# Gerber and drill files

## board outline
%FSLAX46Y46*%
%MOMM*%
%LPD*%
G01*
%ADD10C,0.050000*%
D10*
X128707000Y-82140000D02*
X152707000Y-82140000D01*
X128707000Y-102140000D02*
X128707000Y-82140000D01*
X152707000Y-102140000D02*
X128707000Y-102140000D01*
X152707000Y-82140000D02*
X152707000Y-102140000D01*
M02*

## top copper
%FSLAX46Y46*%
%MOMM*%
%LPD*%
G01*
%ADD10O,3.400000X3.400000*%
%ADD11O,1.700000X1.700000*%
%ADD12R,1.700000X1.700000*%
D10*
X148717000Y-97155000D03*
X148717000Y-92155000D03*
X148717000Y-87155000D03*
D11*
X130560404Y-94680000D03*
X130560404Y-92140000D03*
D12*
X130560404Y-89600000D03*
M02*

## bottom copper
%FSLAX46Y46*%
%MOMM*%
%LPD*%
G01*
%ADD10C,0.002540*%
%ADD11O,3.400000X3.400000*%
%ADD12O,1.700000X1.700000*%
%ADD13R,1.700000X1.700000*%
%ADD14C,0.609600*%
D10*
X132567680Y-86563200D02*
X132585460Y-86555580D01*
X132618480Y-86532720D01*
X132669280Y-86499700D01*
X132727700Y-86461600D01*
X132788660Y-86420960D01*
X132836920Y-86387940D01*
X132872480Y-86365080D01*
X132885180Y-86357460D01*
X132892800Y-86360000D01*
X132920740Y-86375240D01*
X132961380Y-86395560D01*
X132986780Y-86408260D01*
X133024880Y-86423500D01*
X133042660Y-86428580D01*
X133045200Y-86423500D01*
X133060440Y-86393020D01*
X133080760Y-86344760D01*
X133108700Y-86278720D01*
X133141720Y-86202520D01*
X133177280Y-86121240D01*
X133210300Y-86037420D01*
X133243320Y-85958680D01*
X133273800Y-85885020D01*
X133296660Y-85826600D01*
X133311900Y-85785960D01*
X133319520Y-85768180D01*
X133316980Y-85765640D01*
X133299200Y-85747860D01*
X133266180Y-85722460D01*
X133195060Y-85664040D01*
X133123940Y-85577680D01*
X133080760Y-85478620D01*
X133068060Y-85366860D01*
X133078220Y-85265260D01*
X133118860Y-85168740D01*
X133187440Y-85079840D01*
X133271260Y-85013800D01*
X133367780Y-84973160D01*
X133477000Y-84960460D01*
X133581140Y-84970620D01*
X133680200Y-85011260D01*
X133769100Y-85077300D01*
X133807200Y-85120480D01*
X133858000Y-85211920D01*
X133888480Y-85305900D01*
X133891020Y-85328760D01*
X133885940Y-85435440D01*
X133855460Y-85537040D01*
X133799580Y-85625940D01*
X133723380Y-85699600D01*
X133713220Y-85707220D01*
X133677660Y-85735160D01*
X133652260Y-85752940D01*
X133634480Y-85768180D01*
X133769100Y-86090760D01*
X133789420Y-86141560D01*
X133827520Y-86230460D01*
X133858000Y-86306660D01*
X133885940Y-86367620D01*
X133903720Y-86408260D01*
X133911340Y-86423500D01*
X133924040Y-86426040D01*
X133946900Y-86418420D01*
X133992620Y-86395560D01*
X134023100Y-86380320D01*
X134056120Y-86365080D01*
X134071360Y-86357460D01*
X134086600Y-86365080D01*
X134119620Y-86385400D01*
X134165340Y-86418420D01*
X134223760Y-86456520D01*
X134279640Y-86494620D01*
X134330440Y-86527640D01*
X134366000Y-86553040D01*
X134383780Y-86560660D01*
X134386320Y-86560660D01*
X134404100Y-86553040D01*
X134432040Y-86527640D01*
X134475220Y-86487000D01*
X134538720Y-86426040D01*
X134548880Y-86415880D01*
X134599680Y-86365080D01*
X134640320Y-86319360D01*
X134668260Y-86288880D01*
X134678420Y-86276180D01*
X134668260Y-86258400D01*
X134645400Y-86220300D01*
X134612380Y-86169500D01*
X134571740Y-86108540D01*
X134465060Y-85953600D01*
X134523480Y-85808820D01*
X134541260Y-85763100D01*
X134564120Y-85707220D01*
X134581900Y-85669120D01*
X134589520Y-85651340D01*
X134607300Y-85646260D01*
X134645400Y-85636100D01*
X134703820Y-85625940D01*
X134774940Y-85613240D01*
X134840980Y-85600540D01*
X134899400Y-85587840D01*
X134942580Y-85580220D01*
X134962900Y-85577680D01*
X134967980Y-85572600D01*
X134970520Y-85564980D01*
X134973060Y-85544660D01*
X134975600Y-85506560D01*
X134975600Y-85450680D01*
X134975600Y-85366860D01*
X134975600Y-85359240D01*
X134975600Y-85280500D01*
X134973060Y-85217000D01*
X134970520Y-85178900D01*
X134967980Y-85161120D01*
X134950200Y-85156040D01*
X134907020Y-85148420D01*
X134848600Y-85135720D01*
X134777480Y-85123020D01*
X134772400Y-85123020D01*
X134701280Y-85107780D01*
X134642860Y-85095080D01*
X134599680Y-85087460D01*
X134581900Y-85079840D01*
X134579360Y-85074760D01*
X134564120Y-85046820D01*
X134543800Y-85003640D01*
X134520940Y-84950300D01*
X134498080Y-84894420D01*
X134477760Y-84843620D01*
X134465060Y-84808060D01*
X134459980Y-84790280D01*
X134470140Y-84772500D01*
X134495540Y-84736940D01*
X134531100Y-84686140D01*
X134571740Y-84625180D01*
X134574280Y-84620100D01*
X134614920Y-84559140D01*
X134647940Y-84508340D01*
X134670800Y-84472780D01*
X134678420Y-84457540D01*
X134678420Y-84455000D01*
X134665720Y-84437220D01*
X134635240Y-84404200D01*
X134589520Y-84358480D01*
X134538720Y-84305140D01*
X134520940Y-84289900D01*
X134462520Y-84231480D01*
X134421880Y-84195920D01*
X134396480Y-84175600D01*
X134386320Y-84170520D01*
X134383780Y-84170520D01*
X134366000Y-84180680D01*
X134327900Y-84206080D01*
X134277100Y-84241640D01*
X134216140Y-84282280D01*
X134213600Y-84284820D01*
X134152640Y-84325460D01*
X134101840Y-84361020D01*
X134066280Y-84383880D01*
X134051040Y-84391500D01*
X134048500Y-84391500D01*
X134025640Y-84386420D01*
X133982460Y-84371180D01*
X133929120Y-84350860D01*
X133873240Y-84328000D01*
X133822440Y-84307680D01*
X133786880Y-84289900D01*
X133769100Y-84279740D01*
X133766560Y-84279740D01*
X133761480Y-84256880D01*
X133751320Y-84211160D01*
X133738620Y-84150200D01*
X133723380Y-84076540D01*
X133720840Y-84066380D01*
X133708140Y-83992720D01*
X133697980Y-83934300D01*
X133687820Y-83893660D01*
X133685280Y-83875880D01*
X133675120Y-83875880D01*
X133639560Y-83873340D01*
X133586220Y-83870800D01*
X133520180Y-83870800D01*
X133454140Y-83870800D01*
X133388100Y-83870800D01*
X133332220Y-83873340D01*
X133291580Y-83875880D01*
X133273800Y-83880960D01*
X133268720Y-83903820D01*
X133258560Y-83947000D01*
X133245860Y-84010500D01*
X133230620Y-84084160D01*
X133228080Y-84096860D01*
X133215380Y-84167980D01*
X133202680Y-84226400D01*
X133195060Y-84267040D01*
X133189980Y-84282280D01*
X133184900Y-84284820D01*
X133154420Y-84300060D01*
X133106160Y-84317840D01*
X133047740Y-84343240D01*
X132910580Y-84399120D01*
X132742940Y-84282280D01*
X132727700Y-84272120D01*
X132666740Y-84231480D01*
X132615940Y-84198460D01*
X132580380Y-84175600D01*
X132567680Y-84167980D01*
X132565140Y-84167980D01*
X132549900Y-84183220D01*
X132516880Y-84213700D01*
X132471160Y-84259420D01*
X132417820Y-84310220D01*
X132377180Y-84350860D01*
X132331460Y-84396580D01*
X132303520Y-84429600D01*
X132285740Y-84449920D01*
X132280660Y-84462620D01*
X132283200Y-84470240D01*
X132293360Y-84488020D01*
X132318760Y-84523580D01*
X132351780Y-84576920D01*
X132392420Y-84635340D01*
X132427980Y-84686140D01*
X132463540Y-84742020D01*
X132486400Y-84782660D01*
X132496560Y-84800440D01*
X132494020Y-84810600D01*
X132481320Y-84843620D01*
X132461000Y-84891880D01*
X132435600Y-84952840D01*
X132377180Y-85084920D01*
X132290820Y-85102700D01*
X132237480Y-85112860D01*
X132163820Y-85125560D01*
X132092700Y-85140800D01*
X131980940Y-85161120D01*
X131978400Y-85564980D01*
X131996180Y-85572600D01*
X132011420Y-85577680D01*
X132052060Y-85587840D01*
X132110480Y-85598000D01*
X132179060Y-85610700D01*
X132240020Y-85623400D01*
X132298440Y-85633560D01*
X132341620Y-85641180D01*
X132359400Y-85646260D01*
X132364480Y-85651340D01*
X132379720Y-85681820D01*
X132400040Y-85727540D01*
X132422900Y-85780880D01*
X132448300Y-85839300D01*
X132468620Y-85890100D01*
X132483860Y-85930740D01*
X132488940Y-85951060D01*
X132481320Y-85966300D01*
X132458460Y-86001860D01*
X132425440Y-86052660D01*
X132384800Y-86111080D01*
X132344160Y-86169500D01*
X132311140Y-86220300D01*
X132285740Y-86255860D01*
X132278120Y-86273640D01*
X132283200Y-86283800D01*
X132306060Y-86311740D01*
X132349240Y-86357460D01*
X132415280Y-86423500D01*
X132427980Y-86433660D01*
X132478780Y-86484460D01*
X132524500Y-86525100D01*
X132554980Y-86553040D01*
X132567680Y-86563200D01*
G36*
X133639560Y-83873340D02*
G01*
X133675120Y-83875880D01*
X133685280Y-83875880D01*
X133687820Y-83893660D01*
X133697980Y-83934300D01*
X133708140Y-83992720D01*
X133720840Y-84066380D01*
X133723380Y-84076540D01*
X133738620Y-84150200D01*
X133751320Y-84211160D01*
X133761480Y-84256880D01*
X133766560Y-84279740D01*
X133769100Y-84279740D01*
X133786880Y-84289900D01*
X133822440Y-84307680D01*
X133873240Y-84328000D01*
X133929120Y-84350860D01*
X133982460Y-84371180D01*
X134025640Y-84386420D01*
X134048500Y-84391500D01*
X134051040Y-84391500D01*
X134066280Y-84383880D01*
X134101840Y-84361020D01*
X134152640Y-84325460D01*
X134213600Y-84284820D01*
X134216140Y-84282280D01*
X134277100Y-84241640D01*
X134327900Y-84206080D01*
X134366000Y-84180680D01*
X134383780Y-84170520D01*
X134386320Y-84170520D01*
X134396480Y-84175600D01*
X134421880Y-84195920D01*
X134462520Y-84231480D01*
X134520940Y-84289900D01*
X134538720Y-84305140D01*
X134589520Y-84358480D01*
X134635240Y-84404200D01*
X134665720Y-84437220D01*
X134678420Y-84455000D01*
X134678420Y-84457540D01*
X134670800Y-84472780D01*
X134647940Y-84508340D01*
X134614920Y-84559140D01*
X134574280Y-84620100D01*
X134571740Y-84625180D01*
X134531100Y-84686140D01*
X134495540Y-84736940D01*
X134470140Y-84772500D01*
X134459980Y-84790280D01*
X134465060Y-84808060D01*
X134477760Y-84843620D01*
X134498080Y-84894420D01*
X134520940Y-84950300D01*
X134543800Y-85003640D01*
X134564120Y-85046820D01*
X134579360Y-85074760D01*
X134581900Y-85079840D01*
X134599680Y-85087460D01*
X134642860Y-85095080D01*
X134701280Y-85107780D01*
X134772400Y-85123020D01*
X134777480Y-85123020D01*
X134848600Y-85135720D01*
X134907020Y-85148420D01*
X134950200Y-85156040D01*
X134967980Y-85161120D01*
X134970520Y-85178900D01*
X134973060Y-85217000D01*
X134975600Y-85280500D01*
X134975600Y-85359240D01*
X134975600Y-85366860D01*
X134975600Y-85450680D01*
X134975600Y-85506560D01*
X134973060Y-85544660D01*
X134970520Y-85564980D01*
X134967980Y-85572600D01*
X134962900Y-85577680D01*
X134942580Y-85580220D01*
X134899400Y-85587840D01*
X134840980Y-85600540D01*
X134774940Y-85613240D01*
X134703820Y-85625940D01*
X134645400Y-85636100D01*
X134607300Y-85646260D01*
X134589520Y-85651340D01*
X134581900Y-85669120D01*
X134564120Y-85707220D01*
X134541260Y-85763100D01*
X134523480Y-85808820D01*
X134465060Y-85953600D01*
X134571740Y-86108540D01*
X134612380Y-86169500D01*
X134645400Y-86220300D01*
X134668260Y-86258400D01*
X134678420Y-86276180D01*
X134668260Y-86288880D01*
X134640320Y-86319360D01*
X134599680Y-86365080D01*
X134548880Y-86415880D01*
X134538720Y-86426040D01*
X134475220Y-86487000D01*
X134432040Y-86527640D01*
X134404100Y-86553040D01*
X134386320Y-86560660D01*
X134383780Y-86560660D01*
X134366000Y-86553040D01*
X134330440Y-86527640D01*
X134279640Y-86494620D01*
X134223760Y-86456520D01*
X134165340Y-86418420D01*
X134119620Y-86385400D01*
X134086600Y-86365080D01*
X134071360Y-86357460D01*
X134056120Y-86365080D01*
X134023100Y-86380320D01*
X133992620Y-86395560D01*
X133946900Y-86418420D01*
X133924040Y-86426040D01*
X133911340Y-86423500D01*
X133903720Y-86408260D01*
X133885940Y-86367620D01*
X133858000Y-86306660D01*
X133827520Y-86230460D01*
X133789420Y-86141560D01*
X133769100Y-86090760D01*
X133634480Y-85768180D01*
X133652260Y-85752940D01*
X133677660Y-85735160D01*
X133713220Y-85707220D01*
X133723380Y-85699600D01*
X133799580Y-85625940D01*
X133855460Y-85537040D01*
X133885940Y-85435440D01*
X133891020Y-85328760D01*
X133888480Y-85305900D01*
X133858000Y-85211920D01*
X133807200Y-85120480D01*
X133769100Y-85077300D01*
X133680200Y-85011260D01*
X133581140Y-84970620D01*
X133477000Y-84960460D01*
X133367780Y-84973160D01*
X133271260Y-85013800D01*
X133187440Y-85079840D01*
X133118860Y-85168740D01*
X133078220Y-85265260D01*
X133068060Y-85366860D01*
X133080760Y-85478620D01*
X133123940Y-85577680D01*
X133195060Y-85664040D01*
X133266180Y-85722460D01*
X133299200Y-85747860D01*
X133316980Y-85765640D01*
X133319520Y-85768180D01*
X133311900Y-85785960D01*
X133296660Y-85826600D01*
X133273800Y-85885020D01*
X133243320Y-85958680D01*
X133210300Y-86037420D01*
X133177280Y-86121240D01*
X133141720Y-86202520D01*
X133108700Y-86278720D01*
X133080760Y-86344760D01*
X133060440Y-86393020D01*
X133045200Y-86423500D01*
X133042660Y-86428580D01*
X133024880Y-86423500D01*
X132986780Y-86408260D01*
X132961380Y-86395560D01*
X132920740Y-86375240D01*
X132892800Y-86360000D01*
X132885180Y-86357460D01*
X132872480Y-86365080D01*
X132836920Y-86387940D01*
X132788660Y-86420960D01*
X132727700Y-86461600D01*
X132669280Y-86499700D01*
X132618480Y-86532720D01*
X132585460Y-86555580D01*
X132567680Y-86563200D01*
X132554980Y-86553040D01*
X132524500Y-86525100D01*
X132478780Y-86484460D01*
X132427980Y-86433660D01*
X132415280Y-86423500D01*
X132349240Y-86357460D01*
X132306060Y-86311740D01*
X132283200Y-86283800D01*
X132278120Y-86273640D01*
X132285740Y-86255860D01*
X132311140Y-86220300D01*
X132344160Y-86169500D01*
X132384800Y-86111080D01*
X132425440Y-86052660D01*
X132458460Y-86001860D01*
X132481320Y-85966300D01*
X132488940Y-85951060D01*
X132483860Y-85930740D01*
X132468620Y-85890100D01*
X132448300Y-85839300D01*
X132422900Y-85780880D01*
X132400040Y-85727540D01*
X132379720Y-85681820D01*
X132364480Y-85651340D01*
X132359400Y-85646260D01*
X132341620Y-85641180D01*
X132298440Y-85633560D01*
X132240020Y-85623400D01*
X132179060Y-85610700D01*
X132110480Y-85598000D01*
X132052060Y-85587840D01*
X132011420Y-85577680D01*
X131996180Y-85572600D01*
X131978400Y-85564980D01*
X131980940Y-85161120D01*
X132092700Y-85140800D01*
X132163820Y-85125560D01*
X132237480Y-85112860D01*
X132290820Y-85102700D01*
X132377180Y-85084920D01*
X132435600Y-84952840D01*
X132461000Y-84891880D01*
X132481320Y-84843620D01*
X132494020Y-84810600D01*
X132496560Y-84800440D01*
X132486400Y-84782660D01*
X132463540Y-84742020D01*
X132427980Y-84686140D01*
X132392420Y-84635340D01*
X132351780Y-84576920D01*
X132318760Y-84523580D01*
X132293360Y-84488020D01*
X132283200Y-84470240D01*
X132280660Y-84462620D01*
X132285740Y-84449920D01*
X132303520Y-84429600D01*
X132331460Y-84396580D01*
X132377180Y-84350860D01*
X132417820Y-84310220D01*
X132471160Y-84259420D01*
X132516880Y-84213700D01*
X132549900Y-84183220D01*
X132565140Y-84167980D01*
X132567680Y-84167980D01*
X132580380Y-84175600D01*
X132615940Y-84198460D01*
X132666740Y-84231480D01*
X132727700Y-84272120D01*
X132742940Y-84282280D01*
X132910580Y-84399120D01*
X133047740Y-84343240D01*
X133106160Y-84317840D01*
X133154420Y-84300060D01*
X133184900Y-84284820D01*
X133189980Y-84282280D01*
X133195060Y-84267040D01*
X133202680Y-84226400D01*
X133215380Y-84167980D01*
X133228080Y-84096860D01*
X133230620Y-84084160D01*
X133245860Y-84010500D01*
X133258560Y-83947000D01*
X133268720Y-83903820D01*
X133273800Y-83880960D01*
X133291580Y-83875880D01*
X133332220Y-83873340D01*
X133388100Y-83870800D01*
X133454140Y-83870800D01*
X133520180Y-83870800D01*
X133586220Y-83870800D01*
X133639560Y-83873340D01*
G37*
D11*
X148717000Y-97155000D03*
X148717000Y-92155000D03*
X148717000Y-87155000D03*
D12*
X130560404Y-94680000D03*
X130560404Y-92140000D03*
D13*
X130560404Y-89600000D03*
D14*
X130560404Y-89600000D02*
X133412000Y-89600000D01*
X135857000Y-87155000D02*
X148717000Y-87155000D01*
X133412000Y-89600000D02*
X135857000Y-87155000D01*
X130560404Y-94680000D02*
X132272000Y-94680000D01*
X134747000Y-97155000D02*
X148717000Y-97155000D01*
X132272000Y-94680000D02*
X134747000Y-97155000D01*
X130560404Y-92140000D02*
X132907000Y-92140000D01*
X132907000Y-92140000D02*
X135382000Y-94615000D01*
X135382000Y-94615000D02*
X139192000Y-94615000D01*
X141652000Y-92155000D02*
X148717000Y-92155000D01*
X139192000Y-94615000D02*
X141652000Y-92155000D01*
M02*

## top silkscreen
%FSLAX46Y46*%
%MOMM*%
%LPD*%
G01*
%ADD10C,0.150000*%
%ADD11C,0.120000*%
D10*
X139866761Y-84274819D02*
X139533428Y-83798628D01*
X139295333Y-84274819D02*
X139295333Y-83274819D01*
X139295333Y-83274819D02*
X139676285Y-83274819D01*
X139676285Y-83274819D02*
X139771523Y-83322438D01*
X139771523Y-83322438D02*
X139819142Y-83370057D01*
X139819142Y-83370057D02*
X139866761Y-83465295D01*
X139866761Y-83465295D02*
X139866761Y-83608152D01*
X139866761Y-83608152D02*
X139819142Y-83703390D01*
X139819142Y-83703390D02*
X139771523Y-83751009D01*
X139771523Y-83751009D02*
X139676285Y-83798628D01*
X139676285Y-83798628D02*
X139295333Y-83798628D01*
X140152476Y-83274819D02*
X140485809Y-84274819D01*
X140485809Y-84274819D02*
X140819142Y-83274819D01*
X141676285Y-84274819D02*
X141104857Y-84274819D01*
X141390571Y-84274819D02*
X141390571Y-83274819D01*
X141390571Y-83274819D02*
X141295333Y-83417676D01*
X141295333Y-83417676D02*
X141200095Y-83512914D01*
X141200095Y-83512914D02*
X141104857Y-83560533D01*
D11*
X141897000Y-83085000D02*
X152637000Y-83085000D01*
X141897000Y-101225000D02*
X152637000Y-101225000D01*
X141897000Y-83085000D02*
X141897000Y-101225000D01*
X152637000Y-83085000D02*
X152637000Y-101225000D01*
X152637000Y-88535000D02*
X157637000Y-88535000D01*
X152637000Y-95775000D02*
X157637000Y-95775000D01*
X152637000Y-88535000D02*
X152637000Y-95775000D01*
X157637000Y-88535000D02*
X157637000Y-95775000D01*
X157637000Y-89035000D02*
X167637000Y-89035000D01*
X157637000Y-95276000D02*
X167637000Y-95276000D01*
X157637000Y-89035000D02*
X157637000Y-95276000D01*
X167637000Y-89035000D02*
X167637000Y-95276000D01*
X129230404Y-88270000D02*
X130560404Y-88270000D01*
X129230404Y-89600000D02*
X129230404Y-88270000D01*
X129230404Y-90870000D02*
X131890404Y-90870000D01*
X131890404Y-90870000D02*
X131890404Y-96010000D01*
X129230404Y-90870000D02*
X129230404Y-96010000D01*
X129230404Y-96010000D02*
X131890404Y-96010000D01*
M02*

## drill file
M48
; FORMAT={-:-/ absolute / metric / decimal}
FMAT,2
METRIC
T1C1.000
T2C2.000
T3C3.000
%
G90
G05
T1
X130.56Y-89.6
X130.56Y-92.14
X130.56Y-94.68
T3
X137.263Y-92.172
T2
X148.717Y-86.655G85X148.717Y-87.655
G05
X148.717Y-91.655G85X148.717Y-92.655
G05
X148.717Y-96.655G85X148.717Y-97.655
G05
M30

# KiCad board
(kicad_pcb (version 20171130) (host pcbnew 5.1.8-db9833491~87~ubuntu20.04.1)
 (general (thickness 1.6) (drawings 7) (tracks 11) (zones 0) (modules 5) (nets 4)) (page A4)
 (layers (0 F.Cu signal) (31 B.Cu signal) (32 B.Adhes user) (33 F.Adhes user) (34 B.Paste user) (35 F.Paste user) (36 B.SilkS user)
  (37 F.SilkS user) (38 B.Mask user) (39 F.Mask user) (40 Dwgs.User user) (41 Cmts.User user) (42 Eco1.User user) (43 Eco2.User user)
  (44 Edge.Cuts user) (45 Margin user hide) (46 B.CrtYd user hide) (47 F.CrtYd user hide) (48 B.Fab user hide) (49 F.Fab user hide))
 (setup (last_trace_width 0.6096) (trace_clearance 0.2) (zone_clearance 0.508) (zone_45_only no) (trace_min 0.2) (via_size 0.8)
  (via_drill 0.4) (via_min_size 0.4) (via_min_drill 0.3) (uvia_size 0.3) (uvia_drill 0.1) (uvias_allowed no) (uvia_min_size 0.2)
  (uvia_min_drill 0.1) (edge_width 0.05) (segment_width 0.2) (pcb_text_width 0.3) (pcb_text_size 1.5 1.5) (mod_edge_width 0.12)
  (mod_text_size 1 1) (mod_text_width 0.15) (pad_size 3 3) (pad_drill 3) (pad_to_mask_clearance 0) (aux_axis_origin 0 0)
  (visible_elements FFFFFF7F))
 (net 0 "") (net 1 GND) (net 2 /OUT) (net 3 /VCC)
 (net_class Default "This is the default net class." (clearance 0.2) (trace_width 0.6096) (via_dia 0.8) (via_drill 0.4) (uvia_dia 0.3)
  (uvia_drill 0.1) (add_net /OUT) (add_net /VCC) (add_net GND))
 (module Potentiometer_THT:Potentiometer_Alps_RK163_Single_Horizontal (layer F.Cu) (at 148.717 97.155)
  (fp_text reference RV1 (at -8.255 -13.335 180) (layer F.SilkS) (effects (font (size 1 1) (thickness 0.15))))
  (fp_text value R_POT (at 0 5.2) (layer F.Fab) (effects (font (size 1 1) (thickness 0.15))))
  (fp_line (start -6.82 -14.07) (end 3.92 -14.07) (layer F.SilkS) (width 0.12))
  (fp_line (start -6.82 4.07) (end 3.92 4.07) (layer F.SilkS) (width 0.12))
  (fp_line (start -6.82 -14.07) (end -6.82 4.07) (layer F.SilkS) (width 0.12))
  (fp_line (start 3.92 -14.07) (end 3.92 4.07) (layer F.SilkS) (width 0.12))
  (fp_line (start 3.92 -8.62) (end 8.92 -8.62) (layer F.SilkS) (width 0.12))
  (fp_line (start 3.92 -1.38) (end 8.92 -1.38) (layer F.SilkS) (width 0.12))
  (fp_line (start 3.92 -8.62) (end 3.92 -1.38) (layer F.SilkS) (width 0.12))
  (fp_line (start 8.92 -8.62) (end 8.92 -1.38) (layer F.SilkS) (width 0.12))
  (fp_line (start 8.92 -8.12) (end 18.92 -8.12) (layer F.SilkS) (width 0.12))
  (fp_line (start 8.92 -1.879) (end 18.92 -1.879) (layer F.SilkS) (width 0.12))
  (fp_line (start 8.92 -8.12) (end 8.92 -1.879) (layer F.SilkS) (width 0.12))
  (fp_line (start 18.92 -8.12) (end 18.92 -1.879) (layer F.SilkS) (width 0.12))
  (pad 1 thru_hole oval (at 0 0) (size 3.4 3.4) (drill oval 2 3) (layers *.Cu *.Mask) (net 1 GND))
  (pad 2 thru_hole oval (at 0 -5) (size 3.4 3.4) (drill oval 2 3) (layers *.Cu *.Mask) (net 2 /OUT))
  (pad 3 thru_hole oval (at 0 -10) (size 3.4 3.4) (drill oval 2 3) (layers *.Cu *.Mask) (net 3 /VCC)))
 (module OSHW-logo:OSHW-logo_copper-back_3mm (layer B.Cu) (at 133.477 85.217 180)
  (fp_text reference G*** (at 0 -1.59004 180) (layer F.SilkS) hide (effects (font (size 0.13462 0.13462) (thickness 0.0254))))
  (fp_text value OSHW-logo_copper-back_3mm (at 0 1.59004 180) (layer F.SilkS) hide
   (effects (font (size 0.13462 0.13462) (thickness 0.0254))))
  (fp_poly
   (pts (xy 0.90932 -1.3462) (xy 0.89154 -1.33858) (xy 0.85852 -1.31572) (xy 0.80772 -1.2827) (xy 0.7493 -1.2446) (xy 0.68834 -1.20396)
    (xy 0.64008 -1.17094) (xy 0.60452 -1.14808) (xy 0.59182 -1.14046) (xy 0.5842 -1.143) (xy 0.55626 -1.15824) (xy 0.51562 -1.17856)
    (xy 0.49022 -1.19126) (xy 0.45212 -1.2065) (xy 0.43434 -1.21158) (xy 0.4318 -1.2065) (xy 0.41656 -1.17602) (xy 0.39624 -1.12776)
    (xy 0.3683 -1.06172) (xy 0.33528 -0.98552) (xy 0.29972 -0.90424) (xy 0.2667 -0.82042) (xy 0.23368 -0.74168) (xy 0.2032 -0.66802)
    (xy 0.18034 -0.6096) (xy 0.1651 -0.56896) (xy 0.15748 -0.55118) (xy 0.16002 -0.54864) (xy 0.1778 -0.53086) (xy 0.21082 -0.50546)
    (xy 0.28194 -0.44704) (xy 0.35306 -0.36068) (xy 0.39624 -0.26162) (xy 0.40894 -0.14986) (xy 0.39878 -0.04826) (xy 0.35814 0.04826)
    (xy 0.28956 0.13716) (xy 0.20574 0.2032) (xy 0.10922 0.24384) (xy 0 0.25654) (xy -0.10414 0.24638) (xy -0.2032 0.20574)
    (xy -0.2921 0.1397) (xy -0.3302 0.09652) (xy -0.381 0.00508) (xy -0.41148 -0.0889) (xy -0.41402 -0.11176) (xy -0.40894 -0.21844)
    (xy -0.37846 -0.32004) (xy -0.32258 -0.40894) (xy -0.24638 -0.4826) (xy -0.23622 -0.49022) (xy -0.20066 -0.51816) (xy -0.17526 -0.53594)
    (xy -0.15748 -0.55118) (xy -0.2921 -0.87376) (xy -0.31242 -0.92456) (xy -0.35052 -1.01346) (xy -0.381 -1.08966) (xy -0.40894 -1.15062)
    (xy -0.42672 -1.19126) (xy -0.43434 -1.2065) (xy -0.44704 -1.20904) (xy -0.4699 -1.20142) (xy -0.51562 -1.17856) (xy -0.5461 -1.16332)
    (xy -0.57912 -1.14808) (xy -0.59436 -1.14046) (xy -0.6096 -1.14808) (xy -0.64262 -1.1684) (xy -0.68834 -1.20142) (xy -0.74676 -1.23952)
    (xy -0.80264 -1.27762) (xy -0.85344 -1.31064) (xy -0.889 -1.33604) (xy -0.90678 -1.34366) (xy -0.90932 -1.34366) (xy -0.9271 -1.33604)
    (xy -0.95504 -1.31064) (xy -0.99822 -1.27) (xy -1.06172 -1.20904) (xy -1.07188 -1.19888) (xy -1.12268 -1.14808) (xy -1.16332 -1.10236)
    (xy -1.19126 -1.07188) (xy -1.20142 -1.05918) (xy -1.19126 -1.0414) (xy -1.1684 -1.0033) (xy -1.13538 -0.9525) (xy -1.09474 -0.89154)
    (xy -0.98806 -0.7366) (xy -1.04648 -0.59182) (xy -1.06426 -0.5461) (xy -1.08712 -0.49022) (xy -1.1049 -0.45212) (xy -1.11252 -0.43434)
    (xy -1.1303 -0.42926) (xy -1.1684 -0.4191) (xy -1.22682 -0.40894) (xy -1.29794 -0.39624) (xy -1.36398 -0.38354) (xy -1.4224 -0.37084)
    (xy -1.46558 -0.36322) (xy -1.4859 -0.36068) (xy -1.49098 -0.3556) (xy -1.49352 -0.34798) (xy -1.49606 -0.32766) (xy -1.4986 -0.28956)
    (xy -1.4986 -0.23368) (xy -1.4986 -0.14986) (xy -1.4986 -0.14224) (xy -1.4986 -0.0635) (xy -1.49606 0) (xy -1.49352 0.0381)
    (xy -1.49098 0.05588) (xy -1.4732 0.06096) (xy -1.43002 0.06858) (xy -1.3716 0.08128) (xy -1.30048 0.09398) (xy -1.2954 0.09398)
    (xy -1.22428 0.10922) (xy -1.16586 0.12192) (xy -1.12268 0.12954) (xy -1.1049 0.13716) (xy -1.10236 0.14224) (xy -1.08712 0.17018)
    (xy -1.0668 0.21336) (xy -1.04394 0.2667) (xy -1.02108 0.32258) (xy -1.00076 0.37338) (xy -0.98806 0.40894) (xy -0.98298 0.42672)
    (xy -0.99314 0.4445) (xy -1.01854 0.48006) (xy -1.0541 0.53086) (xy -1.09474 0.59182) (xy -1.09728 0.5969) (xy -1.13792 0.65786)
    (xy -1.17094 0.70866) (xy -1.1938 0.74422) (xy -1.20142 0.75946) (xy -1.20142 0.762) (xy -1.18872 0.77978) (xy -1.15824 0.8128)
    (xy -1.11252 0.85852) (xy -1.06172 0.91186) (xy -1.04394 0.9271) (xy -0.98552 0.98552) (xy -0.94488 1.02108) (xy -0.91948 1.0414)
    (xy -0.90932 1.04648) (xy -0.90678 1.04648) (xy -0.889 1.03632) (xy -0.8509 1.01092) (xy -0.8001 0.97536) (xy -0.73914 0.93472)
    (xy -0.7366 0.93218) (xy -0.67564 0.89154) (xy -0.62484 0.85598) (xy -0.58928 0.83312) (xy -0.57404 0.8255) (xy -0.5715 0.8255)
    (xy -0.54864 0.83058) (xy -0.50546 0.84582) (xy -0.45212 0.86614) (xy -0.39624 0.889) (xy -0.34544 0.90932) (xy -0.30988 0.9271)
    (xy -0.2921 0.93726) (xy -0.28956 0.93726) (xy -0.28448 0.96012) (xy -0.27432 1.00584) (xy -0.26162 1.0668) (xy -0.24638 1.14046)
    (xy -0.24384 1.15062) (xy -0.23114 1.22428) (xy -0.22098 1.2827) (xy -0.21082 1.32334) (xy -0.20828 1.34112) (xy -0.19812 1.34112)
    (xy -0.16256 1.34366) (xy -0.10922 1.3462) (xy -0.04318 1.3462) (xy 0.02286 1.3462) (xy 0.0889 1.3462) (xy 0.14478 1.34366)
    (xy 0.18542 1.34112) (xy 0.2032 1.33604) (xy 0.20828 1.31318) (xy 0.21844 1.27) (xy 0.23114 1.2065) (xy 0.24638 1.13284)
    (xy 0.24892 1.12014) (xy 0.26162 1.04902) (xy 0.27432 0.9906) (xy 0.28194 0.94996) (xy 0.28702 0.93472) (xy 0.2921 0.93218)
    (xy 0.32258 0.91694) (xy 0.37084 0.89916) (xy 0.42926 0.87376) (xy 0.56642 0.81788) (xy 0.73406 0.93472) (xy 0.7493 0.94488)
    (xy 0.81026 0.98552) (xy 0.86106 1.01854) (xy 0.89662 1.0414) (xy 0.90932 1.04902) (xy 0.91186 1.04902) (xy 0.9271 1.03378)
    (xy 0.96012 1.0033) (xy 1.00584 0.95758) (xy 1.05918 0.90678) (xy 1.09982 0.86614) (xy 1.14554 0.82042) (xy 1.17348 0.7874)
    (xy 1.19126 0.76708) (xy 1.19634 0.75438) (xy 1.1938 0.74676) (xy 1.18364 0.72898) (xy 1.15824 0.69342) (xy 1.12522 0.64008)
    (xy 1.08458 0.58166) (xy 1.04902 0.53086) (xy 1.01346 0.47498) (xy 0.9906 0.43434) (xy 0.98044 0.41656) (xy 0.98298 0.4064)
    (xy 0.99568 0.37338) (xy 1.016 0.32512) (xy 1.0414 0.26416) (xy 1.09982 0.13208) (xy 1.18618 0.1143) (xy 1.23952 0.10414)
    (xy 1.31318 0.09144) (xy 1.3843 0.0762) (xy 1.49606 0.05588) (xy 1.4986 -0.34798) (xy 1.48082 -0.3556) (xy 1.46558 -0.36068)
    (xy 1.42494 -0.37084) (xy 1.36652 -0.381) (xy 1.29794 -0.3937) (xy 1.23698 -0.4064) (xy 1.17856 -0.41656) (xy 1.13538 -0.42418)
    (xy 1.1176 -0.42926) (xy 1.11252 -0.43434) (xy 1.09728 -0.46482) (xy 1.07696 -0.51054) (xy 1.0541 -0.56388) (xy 1.0287 -0.6223)
    (xy 1.00838 -0.6731) (xy 0.99314 -0.71374) (xy 0.98806 -0.73406) (xy 0.99568 -0.7493) (xy 1.01854 -0.78486) (xy 1.05156 -0.83566)
    (xy 1.0922 -0.89408) (xy 1.13284 -0.9525) (xy 1.16586 -1.0033) (xy 1.19126 -1.03886) (xy 1.19888 -1.05664) (xy 1.1938 -1.0668)
    (xy 1.17094 -1.09474) (xy 1.12776 -1.14046) (xy 1.06172 -1.2065) (xy 1.04902 -1.21666) (xy 0.99822 -1.26746) (xy 0.9525 -1.3081)
    (xy 0.92202 -1.33604) (xy 0.90932 -1.3462))
   (layer B.Cu) (width 0.00254)))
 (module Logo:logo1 (layer B.Cu) (at 139.192 99.06 180)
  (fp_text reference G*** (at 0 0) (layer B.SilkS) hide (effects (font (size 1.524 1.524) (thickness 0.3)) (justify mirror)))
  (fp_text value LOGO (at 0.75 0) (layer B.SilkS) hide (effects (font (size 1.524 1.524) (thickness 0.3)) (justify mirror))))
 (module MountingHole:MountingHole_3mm (layer F.Cu) (at 131.682721 90.237113)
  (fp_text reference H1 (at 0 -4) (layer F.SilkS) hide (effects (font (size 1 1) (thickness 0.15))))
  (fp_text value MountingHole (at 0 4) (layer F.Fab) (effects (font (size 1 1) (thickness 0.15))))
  (pad "" np_thru_hole circle (at 5.58 1.935) (size 3 3) (drill 3) (layers *.Cu *.Mask)))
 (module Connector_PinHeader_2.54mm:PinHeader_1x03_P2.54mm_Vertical (layer F.Cu) (at 130.560404 89.6)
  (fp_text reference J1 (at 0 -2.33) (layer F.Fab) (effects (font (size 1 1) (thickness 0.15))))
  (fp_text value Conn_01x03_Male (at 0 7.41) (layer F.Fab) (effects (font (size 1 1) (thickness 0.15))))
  (fp_line (start -1.33 -1.33) (end 0 -1.33) (layer F.SilkS) (width 0.12))
  (fp_line (start -1.33 0) (end -1.33 -1.33) (layer F.SilkS) (width 0.12))
  (fp_line (start -1.33 1.27) (end 1.33 1.27) (layer F.SilkS) (width 0.12))
  (fp_line (start 1.33 1.27) (end 1.33 6.41) (layer F.SilkS) (width 0.12))
  (fp_line (start -1.33 1.27) (end -1.33 6.41) (layer F.SilkS) (width 0.12))
  (fp_line (start -1.33 6.41) (end 1.33 6.41) (layer F.SilkS) (width 0.12))
  (pad 3 thru_hole oval (at 0 5.08) (size 1.7 1.7) (drill 1) (layers *.Cu *.Mask) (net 1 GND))
  (pad 2 thru_hole oval (at 0 2.54) (size 1.7 1.7) (drill 1) (layers *.Cu *.Mask) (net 2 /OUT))
  (pad 1 thru_hole rect (at 0 0) (size 1.7 1.7) (drill 1) (layers *.Cu *.Mask) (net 3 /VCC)))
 (gr_line (start 128.707 82.14) (end 152.707 82.14) (layer Edge.Cuts) (width 0.05))
 (gr_line (start 128.707 102.14) (end 128.707 82.14) (layer Edge.Cuts) (width 0.05))
 (gr_line (start 152.707 102.14) (end 128.707 102.14) (layer Edge.Cuts) (width 0.05))
 (gr_line (start 152.707 82.14) (end 152.707 102.14) (layer Edge.Cuts) (width 0.05))
 (segment (start 130.560404 89.6) (end 133.412 89.6) (width 0.6096) (layer B.Cu) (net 3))
 (segment (start 135.857 87.155) (end 148.717 87.155) (width 0.6096) (layer B.Cu) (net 3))
 (segment (start 133.412 89.6) (end 135.857 87.155) (width 0.6096) (layer B.Cu) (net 3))
 (segment (start 130.560404 94.68) (end 132.272 94.68) (width 0.6096) (layer B.Cu) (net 1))
 (segment (start 134.747 97.155) (end 148.717 97.155) (width 0.6096) (layer B.Cu) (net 1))
 (segment (start 132.272 94.68) (end 134.747 97.155) (width 0.6096) (layer B.Cu) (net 1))
 (segment (start 130.560404 92.14) (end 132.907 92.14) (width 0.6096) (layer B.Cu) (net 2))
 (segment (start 132.907 92.14) (end 135.382 94.615) (width 0.6096) (layer B.Cu) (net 2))
 (segment (start 135.382 94.615) (end 139.192 94.615) (width 0.6096) (layer B.Cu) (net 2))
 (segment (start 141.652 92.155) (end 148.717 92.155) (width 0.6096) (layer B.Cu) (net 2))
 (segment (start 139.192 94.615) (end 141.652 92.155) (width 0.6096) (layer B.Cu) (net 2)))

